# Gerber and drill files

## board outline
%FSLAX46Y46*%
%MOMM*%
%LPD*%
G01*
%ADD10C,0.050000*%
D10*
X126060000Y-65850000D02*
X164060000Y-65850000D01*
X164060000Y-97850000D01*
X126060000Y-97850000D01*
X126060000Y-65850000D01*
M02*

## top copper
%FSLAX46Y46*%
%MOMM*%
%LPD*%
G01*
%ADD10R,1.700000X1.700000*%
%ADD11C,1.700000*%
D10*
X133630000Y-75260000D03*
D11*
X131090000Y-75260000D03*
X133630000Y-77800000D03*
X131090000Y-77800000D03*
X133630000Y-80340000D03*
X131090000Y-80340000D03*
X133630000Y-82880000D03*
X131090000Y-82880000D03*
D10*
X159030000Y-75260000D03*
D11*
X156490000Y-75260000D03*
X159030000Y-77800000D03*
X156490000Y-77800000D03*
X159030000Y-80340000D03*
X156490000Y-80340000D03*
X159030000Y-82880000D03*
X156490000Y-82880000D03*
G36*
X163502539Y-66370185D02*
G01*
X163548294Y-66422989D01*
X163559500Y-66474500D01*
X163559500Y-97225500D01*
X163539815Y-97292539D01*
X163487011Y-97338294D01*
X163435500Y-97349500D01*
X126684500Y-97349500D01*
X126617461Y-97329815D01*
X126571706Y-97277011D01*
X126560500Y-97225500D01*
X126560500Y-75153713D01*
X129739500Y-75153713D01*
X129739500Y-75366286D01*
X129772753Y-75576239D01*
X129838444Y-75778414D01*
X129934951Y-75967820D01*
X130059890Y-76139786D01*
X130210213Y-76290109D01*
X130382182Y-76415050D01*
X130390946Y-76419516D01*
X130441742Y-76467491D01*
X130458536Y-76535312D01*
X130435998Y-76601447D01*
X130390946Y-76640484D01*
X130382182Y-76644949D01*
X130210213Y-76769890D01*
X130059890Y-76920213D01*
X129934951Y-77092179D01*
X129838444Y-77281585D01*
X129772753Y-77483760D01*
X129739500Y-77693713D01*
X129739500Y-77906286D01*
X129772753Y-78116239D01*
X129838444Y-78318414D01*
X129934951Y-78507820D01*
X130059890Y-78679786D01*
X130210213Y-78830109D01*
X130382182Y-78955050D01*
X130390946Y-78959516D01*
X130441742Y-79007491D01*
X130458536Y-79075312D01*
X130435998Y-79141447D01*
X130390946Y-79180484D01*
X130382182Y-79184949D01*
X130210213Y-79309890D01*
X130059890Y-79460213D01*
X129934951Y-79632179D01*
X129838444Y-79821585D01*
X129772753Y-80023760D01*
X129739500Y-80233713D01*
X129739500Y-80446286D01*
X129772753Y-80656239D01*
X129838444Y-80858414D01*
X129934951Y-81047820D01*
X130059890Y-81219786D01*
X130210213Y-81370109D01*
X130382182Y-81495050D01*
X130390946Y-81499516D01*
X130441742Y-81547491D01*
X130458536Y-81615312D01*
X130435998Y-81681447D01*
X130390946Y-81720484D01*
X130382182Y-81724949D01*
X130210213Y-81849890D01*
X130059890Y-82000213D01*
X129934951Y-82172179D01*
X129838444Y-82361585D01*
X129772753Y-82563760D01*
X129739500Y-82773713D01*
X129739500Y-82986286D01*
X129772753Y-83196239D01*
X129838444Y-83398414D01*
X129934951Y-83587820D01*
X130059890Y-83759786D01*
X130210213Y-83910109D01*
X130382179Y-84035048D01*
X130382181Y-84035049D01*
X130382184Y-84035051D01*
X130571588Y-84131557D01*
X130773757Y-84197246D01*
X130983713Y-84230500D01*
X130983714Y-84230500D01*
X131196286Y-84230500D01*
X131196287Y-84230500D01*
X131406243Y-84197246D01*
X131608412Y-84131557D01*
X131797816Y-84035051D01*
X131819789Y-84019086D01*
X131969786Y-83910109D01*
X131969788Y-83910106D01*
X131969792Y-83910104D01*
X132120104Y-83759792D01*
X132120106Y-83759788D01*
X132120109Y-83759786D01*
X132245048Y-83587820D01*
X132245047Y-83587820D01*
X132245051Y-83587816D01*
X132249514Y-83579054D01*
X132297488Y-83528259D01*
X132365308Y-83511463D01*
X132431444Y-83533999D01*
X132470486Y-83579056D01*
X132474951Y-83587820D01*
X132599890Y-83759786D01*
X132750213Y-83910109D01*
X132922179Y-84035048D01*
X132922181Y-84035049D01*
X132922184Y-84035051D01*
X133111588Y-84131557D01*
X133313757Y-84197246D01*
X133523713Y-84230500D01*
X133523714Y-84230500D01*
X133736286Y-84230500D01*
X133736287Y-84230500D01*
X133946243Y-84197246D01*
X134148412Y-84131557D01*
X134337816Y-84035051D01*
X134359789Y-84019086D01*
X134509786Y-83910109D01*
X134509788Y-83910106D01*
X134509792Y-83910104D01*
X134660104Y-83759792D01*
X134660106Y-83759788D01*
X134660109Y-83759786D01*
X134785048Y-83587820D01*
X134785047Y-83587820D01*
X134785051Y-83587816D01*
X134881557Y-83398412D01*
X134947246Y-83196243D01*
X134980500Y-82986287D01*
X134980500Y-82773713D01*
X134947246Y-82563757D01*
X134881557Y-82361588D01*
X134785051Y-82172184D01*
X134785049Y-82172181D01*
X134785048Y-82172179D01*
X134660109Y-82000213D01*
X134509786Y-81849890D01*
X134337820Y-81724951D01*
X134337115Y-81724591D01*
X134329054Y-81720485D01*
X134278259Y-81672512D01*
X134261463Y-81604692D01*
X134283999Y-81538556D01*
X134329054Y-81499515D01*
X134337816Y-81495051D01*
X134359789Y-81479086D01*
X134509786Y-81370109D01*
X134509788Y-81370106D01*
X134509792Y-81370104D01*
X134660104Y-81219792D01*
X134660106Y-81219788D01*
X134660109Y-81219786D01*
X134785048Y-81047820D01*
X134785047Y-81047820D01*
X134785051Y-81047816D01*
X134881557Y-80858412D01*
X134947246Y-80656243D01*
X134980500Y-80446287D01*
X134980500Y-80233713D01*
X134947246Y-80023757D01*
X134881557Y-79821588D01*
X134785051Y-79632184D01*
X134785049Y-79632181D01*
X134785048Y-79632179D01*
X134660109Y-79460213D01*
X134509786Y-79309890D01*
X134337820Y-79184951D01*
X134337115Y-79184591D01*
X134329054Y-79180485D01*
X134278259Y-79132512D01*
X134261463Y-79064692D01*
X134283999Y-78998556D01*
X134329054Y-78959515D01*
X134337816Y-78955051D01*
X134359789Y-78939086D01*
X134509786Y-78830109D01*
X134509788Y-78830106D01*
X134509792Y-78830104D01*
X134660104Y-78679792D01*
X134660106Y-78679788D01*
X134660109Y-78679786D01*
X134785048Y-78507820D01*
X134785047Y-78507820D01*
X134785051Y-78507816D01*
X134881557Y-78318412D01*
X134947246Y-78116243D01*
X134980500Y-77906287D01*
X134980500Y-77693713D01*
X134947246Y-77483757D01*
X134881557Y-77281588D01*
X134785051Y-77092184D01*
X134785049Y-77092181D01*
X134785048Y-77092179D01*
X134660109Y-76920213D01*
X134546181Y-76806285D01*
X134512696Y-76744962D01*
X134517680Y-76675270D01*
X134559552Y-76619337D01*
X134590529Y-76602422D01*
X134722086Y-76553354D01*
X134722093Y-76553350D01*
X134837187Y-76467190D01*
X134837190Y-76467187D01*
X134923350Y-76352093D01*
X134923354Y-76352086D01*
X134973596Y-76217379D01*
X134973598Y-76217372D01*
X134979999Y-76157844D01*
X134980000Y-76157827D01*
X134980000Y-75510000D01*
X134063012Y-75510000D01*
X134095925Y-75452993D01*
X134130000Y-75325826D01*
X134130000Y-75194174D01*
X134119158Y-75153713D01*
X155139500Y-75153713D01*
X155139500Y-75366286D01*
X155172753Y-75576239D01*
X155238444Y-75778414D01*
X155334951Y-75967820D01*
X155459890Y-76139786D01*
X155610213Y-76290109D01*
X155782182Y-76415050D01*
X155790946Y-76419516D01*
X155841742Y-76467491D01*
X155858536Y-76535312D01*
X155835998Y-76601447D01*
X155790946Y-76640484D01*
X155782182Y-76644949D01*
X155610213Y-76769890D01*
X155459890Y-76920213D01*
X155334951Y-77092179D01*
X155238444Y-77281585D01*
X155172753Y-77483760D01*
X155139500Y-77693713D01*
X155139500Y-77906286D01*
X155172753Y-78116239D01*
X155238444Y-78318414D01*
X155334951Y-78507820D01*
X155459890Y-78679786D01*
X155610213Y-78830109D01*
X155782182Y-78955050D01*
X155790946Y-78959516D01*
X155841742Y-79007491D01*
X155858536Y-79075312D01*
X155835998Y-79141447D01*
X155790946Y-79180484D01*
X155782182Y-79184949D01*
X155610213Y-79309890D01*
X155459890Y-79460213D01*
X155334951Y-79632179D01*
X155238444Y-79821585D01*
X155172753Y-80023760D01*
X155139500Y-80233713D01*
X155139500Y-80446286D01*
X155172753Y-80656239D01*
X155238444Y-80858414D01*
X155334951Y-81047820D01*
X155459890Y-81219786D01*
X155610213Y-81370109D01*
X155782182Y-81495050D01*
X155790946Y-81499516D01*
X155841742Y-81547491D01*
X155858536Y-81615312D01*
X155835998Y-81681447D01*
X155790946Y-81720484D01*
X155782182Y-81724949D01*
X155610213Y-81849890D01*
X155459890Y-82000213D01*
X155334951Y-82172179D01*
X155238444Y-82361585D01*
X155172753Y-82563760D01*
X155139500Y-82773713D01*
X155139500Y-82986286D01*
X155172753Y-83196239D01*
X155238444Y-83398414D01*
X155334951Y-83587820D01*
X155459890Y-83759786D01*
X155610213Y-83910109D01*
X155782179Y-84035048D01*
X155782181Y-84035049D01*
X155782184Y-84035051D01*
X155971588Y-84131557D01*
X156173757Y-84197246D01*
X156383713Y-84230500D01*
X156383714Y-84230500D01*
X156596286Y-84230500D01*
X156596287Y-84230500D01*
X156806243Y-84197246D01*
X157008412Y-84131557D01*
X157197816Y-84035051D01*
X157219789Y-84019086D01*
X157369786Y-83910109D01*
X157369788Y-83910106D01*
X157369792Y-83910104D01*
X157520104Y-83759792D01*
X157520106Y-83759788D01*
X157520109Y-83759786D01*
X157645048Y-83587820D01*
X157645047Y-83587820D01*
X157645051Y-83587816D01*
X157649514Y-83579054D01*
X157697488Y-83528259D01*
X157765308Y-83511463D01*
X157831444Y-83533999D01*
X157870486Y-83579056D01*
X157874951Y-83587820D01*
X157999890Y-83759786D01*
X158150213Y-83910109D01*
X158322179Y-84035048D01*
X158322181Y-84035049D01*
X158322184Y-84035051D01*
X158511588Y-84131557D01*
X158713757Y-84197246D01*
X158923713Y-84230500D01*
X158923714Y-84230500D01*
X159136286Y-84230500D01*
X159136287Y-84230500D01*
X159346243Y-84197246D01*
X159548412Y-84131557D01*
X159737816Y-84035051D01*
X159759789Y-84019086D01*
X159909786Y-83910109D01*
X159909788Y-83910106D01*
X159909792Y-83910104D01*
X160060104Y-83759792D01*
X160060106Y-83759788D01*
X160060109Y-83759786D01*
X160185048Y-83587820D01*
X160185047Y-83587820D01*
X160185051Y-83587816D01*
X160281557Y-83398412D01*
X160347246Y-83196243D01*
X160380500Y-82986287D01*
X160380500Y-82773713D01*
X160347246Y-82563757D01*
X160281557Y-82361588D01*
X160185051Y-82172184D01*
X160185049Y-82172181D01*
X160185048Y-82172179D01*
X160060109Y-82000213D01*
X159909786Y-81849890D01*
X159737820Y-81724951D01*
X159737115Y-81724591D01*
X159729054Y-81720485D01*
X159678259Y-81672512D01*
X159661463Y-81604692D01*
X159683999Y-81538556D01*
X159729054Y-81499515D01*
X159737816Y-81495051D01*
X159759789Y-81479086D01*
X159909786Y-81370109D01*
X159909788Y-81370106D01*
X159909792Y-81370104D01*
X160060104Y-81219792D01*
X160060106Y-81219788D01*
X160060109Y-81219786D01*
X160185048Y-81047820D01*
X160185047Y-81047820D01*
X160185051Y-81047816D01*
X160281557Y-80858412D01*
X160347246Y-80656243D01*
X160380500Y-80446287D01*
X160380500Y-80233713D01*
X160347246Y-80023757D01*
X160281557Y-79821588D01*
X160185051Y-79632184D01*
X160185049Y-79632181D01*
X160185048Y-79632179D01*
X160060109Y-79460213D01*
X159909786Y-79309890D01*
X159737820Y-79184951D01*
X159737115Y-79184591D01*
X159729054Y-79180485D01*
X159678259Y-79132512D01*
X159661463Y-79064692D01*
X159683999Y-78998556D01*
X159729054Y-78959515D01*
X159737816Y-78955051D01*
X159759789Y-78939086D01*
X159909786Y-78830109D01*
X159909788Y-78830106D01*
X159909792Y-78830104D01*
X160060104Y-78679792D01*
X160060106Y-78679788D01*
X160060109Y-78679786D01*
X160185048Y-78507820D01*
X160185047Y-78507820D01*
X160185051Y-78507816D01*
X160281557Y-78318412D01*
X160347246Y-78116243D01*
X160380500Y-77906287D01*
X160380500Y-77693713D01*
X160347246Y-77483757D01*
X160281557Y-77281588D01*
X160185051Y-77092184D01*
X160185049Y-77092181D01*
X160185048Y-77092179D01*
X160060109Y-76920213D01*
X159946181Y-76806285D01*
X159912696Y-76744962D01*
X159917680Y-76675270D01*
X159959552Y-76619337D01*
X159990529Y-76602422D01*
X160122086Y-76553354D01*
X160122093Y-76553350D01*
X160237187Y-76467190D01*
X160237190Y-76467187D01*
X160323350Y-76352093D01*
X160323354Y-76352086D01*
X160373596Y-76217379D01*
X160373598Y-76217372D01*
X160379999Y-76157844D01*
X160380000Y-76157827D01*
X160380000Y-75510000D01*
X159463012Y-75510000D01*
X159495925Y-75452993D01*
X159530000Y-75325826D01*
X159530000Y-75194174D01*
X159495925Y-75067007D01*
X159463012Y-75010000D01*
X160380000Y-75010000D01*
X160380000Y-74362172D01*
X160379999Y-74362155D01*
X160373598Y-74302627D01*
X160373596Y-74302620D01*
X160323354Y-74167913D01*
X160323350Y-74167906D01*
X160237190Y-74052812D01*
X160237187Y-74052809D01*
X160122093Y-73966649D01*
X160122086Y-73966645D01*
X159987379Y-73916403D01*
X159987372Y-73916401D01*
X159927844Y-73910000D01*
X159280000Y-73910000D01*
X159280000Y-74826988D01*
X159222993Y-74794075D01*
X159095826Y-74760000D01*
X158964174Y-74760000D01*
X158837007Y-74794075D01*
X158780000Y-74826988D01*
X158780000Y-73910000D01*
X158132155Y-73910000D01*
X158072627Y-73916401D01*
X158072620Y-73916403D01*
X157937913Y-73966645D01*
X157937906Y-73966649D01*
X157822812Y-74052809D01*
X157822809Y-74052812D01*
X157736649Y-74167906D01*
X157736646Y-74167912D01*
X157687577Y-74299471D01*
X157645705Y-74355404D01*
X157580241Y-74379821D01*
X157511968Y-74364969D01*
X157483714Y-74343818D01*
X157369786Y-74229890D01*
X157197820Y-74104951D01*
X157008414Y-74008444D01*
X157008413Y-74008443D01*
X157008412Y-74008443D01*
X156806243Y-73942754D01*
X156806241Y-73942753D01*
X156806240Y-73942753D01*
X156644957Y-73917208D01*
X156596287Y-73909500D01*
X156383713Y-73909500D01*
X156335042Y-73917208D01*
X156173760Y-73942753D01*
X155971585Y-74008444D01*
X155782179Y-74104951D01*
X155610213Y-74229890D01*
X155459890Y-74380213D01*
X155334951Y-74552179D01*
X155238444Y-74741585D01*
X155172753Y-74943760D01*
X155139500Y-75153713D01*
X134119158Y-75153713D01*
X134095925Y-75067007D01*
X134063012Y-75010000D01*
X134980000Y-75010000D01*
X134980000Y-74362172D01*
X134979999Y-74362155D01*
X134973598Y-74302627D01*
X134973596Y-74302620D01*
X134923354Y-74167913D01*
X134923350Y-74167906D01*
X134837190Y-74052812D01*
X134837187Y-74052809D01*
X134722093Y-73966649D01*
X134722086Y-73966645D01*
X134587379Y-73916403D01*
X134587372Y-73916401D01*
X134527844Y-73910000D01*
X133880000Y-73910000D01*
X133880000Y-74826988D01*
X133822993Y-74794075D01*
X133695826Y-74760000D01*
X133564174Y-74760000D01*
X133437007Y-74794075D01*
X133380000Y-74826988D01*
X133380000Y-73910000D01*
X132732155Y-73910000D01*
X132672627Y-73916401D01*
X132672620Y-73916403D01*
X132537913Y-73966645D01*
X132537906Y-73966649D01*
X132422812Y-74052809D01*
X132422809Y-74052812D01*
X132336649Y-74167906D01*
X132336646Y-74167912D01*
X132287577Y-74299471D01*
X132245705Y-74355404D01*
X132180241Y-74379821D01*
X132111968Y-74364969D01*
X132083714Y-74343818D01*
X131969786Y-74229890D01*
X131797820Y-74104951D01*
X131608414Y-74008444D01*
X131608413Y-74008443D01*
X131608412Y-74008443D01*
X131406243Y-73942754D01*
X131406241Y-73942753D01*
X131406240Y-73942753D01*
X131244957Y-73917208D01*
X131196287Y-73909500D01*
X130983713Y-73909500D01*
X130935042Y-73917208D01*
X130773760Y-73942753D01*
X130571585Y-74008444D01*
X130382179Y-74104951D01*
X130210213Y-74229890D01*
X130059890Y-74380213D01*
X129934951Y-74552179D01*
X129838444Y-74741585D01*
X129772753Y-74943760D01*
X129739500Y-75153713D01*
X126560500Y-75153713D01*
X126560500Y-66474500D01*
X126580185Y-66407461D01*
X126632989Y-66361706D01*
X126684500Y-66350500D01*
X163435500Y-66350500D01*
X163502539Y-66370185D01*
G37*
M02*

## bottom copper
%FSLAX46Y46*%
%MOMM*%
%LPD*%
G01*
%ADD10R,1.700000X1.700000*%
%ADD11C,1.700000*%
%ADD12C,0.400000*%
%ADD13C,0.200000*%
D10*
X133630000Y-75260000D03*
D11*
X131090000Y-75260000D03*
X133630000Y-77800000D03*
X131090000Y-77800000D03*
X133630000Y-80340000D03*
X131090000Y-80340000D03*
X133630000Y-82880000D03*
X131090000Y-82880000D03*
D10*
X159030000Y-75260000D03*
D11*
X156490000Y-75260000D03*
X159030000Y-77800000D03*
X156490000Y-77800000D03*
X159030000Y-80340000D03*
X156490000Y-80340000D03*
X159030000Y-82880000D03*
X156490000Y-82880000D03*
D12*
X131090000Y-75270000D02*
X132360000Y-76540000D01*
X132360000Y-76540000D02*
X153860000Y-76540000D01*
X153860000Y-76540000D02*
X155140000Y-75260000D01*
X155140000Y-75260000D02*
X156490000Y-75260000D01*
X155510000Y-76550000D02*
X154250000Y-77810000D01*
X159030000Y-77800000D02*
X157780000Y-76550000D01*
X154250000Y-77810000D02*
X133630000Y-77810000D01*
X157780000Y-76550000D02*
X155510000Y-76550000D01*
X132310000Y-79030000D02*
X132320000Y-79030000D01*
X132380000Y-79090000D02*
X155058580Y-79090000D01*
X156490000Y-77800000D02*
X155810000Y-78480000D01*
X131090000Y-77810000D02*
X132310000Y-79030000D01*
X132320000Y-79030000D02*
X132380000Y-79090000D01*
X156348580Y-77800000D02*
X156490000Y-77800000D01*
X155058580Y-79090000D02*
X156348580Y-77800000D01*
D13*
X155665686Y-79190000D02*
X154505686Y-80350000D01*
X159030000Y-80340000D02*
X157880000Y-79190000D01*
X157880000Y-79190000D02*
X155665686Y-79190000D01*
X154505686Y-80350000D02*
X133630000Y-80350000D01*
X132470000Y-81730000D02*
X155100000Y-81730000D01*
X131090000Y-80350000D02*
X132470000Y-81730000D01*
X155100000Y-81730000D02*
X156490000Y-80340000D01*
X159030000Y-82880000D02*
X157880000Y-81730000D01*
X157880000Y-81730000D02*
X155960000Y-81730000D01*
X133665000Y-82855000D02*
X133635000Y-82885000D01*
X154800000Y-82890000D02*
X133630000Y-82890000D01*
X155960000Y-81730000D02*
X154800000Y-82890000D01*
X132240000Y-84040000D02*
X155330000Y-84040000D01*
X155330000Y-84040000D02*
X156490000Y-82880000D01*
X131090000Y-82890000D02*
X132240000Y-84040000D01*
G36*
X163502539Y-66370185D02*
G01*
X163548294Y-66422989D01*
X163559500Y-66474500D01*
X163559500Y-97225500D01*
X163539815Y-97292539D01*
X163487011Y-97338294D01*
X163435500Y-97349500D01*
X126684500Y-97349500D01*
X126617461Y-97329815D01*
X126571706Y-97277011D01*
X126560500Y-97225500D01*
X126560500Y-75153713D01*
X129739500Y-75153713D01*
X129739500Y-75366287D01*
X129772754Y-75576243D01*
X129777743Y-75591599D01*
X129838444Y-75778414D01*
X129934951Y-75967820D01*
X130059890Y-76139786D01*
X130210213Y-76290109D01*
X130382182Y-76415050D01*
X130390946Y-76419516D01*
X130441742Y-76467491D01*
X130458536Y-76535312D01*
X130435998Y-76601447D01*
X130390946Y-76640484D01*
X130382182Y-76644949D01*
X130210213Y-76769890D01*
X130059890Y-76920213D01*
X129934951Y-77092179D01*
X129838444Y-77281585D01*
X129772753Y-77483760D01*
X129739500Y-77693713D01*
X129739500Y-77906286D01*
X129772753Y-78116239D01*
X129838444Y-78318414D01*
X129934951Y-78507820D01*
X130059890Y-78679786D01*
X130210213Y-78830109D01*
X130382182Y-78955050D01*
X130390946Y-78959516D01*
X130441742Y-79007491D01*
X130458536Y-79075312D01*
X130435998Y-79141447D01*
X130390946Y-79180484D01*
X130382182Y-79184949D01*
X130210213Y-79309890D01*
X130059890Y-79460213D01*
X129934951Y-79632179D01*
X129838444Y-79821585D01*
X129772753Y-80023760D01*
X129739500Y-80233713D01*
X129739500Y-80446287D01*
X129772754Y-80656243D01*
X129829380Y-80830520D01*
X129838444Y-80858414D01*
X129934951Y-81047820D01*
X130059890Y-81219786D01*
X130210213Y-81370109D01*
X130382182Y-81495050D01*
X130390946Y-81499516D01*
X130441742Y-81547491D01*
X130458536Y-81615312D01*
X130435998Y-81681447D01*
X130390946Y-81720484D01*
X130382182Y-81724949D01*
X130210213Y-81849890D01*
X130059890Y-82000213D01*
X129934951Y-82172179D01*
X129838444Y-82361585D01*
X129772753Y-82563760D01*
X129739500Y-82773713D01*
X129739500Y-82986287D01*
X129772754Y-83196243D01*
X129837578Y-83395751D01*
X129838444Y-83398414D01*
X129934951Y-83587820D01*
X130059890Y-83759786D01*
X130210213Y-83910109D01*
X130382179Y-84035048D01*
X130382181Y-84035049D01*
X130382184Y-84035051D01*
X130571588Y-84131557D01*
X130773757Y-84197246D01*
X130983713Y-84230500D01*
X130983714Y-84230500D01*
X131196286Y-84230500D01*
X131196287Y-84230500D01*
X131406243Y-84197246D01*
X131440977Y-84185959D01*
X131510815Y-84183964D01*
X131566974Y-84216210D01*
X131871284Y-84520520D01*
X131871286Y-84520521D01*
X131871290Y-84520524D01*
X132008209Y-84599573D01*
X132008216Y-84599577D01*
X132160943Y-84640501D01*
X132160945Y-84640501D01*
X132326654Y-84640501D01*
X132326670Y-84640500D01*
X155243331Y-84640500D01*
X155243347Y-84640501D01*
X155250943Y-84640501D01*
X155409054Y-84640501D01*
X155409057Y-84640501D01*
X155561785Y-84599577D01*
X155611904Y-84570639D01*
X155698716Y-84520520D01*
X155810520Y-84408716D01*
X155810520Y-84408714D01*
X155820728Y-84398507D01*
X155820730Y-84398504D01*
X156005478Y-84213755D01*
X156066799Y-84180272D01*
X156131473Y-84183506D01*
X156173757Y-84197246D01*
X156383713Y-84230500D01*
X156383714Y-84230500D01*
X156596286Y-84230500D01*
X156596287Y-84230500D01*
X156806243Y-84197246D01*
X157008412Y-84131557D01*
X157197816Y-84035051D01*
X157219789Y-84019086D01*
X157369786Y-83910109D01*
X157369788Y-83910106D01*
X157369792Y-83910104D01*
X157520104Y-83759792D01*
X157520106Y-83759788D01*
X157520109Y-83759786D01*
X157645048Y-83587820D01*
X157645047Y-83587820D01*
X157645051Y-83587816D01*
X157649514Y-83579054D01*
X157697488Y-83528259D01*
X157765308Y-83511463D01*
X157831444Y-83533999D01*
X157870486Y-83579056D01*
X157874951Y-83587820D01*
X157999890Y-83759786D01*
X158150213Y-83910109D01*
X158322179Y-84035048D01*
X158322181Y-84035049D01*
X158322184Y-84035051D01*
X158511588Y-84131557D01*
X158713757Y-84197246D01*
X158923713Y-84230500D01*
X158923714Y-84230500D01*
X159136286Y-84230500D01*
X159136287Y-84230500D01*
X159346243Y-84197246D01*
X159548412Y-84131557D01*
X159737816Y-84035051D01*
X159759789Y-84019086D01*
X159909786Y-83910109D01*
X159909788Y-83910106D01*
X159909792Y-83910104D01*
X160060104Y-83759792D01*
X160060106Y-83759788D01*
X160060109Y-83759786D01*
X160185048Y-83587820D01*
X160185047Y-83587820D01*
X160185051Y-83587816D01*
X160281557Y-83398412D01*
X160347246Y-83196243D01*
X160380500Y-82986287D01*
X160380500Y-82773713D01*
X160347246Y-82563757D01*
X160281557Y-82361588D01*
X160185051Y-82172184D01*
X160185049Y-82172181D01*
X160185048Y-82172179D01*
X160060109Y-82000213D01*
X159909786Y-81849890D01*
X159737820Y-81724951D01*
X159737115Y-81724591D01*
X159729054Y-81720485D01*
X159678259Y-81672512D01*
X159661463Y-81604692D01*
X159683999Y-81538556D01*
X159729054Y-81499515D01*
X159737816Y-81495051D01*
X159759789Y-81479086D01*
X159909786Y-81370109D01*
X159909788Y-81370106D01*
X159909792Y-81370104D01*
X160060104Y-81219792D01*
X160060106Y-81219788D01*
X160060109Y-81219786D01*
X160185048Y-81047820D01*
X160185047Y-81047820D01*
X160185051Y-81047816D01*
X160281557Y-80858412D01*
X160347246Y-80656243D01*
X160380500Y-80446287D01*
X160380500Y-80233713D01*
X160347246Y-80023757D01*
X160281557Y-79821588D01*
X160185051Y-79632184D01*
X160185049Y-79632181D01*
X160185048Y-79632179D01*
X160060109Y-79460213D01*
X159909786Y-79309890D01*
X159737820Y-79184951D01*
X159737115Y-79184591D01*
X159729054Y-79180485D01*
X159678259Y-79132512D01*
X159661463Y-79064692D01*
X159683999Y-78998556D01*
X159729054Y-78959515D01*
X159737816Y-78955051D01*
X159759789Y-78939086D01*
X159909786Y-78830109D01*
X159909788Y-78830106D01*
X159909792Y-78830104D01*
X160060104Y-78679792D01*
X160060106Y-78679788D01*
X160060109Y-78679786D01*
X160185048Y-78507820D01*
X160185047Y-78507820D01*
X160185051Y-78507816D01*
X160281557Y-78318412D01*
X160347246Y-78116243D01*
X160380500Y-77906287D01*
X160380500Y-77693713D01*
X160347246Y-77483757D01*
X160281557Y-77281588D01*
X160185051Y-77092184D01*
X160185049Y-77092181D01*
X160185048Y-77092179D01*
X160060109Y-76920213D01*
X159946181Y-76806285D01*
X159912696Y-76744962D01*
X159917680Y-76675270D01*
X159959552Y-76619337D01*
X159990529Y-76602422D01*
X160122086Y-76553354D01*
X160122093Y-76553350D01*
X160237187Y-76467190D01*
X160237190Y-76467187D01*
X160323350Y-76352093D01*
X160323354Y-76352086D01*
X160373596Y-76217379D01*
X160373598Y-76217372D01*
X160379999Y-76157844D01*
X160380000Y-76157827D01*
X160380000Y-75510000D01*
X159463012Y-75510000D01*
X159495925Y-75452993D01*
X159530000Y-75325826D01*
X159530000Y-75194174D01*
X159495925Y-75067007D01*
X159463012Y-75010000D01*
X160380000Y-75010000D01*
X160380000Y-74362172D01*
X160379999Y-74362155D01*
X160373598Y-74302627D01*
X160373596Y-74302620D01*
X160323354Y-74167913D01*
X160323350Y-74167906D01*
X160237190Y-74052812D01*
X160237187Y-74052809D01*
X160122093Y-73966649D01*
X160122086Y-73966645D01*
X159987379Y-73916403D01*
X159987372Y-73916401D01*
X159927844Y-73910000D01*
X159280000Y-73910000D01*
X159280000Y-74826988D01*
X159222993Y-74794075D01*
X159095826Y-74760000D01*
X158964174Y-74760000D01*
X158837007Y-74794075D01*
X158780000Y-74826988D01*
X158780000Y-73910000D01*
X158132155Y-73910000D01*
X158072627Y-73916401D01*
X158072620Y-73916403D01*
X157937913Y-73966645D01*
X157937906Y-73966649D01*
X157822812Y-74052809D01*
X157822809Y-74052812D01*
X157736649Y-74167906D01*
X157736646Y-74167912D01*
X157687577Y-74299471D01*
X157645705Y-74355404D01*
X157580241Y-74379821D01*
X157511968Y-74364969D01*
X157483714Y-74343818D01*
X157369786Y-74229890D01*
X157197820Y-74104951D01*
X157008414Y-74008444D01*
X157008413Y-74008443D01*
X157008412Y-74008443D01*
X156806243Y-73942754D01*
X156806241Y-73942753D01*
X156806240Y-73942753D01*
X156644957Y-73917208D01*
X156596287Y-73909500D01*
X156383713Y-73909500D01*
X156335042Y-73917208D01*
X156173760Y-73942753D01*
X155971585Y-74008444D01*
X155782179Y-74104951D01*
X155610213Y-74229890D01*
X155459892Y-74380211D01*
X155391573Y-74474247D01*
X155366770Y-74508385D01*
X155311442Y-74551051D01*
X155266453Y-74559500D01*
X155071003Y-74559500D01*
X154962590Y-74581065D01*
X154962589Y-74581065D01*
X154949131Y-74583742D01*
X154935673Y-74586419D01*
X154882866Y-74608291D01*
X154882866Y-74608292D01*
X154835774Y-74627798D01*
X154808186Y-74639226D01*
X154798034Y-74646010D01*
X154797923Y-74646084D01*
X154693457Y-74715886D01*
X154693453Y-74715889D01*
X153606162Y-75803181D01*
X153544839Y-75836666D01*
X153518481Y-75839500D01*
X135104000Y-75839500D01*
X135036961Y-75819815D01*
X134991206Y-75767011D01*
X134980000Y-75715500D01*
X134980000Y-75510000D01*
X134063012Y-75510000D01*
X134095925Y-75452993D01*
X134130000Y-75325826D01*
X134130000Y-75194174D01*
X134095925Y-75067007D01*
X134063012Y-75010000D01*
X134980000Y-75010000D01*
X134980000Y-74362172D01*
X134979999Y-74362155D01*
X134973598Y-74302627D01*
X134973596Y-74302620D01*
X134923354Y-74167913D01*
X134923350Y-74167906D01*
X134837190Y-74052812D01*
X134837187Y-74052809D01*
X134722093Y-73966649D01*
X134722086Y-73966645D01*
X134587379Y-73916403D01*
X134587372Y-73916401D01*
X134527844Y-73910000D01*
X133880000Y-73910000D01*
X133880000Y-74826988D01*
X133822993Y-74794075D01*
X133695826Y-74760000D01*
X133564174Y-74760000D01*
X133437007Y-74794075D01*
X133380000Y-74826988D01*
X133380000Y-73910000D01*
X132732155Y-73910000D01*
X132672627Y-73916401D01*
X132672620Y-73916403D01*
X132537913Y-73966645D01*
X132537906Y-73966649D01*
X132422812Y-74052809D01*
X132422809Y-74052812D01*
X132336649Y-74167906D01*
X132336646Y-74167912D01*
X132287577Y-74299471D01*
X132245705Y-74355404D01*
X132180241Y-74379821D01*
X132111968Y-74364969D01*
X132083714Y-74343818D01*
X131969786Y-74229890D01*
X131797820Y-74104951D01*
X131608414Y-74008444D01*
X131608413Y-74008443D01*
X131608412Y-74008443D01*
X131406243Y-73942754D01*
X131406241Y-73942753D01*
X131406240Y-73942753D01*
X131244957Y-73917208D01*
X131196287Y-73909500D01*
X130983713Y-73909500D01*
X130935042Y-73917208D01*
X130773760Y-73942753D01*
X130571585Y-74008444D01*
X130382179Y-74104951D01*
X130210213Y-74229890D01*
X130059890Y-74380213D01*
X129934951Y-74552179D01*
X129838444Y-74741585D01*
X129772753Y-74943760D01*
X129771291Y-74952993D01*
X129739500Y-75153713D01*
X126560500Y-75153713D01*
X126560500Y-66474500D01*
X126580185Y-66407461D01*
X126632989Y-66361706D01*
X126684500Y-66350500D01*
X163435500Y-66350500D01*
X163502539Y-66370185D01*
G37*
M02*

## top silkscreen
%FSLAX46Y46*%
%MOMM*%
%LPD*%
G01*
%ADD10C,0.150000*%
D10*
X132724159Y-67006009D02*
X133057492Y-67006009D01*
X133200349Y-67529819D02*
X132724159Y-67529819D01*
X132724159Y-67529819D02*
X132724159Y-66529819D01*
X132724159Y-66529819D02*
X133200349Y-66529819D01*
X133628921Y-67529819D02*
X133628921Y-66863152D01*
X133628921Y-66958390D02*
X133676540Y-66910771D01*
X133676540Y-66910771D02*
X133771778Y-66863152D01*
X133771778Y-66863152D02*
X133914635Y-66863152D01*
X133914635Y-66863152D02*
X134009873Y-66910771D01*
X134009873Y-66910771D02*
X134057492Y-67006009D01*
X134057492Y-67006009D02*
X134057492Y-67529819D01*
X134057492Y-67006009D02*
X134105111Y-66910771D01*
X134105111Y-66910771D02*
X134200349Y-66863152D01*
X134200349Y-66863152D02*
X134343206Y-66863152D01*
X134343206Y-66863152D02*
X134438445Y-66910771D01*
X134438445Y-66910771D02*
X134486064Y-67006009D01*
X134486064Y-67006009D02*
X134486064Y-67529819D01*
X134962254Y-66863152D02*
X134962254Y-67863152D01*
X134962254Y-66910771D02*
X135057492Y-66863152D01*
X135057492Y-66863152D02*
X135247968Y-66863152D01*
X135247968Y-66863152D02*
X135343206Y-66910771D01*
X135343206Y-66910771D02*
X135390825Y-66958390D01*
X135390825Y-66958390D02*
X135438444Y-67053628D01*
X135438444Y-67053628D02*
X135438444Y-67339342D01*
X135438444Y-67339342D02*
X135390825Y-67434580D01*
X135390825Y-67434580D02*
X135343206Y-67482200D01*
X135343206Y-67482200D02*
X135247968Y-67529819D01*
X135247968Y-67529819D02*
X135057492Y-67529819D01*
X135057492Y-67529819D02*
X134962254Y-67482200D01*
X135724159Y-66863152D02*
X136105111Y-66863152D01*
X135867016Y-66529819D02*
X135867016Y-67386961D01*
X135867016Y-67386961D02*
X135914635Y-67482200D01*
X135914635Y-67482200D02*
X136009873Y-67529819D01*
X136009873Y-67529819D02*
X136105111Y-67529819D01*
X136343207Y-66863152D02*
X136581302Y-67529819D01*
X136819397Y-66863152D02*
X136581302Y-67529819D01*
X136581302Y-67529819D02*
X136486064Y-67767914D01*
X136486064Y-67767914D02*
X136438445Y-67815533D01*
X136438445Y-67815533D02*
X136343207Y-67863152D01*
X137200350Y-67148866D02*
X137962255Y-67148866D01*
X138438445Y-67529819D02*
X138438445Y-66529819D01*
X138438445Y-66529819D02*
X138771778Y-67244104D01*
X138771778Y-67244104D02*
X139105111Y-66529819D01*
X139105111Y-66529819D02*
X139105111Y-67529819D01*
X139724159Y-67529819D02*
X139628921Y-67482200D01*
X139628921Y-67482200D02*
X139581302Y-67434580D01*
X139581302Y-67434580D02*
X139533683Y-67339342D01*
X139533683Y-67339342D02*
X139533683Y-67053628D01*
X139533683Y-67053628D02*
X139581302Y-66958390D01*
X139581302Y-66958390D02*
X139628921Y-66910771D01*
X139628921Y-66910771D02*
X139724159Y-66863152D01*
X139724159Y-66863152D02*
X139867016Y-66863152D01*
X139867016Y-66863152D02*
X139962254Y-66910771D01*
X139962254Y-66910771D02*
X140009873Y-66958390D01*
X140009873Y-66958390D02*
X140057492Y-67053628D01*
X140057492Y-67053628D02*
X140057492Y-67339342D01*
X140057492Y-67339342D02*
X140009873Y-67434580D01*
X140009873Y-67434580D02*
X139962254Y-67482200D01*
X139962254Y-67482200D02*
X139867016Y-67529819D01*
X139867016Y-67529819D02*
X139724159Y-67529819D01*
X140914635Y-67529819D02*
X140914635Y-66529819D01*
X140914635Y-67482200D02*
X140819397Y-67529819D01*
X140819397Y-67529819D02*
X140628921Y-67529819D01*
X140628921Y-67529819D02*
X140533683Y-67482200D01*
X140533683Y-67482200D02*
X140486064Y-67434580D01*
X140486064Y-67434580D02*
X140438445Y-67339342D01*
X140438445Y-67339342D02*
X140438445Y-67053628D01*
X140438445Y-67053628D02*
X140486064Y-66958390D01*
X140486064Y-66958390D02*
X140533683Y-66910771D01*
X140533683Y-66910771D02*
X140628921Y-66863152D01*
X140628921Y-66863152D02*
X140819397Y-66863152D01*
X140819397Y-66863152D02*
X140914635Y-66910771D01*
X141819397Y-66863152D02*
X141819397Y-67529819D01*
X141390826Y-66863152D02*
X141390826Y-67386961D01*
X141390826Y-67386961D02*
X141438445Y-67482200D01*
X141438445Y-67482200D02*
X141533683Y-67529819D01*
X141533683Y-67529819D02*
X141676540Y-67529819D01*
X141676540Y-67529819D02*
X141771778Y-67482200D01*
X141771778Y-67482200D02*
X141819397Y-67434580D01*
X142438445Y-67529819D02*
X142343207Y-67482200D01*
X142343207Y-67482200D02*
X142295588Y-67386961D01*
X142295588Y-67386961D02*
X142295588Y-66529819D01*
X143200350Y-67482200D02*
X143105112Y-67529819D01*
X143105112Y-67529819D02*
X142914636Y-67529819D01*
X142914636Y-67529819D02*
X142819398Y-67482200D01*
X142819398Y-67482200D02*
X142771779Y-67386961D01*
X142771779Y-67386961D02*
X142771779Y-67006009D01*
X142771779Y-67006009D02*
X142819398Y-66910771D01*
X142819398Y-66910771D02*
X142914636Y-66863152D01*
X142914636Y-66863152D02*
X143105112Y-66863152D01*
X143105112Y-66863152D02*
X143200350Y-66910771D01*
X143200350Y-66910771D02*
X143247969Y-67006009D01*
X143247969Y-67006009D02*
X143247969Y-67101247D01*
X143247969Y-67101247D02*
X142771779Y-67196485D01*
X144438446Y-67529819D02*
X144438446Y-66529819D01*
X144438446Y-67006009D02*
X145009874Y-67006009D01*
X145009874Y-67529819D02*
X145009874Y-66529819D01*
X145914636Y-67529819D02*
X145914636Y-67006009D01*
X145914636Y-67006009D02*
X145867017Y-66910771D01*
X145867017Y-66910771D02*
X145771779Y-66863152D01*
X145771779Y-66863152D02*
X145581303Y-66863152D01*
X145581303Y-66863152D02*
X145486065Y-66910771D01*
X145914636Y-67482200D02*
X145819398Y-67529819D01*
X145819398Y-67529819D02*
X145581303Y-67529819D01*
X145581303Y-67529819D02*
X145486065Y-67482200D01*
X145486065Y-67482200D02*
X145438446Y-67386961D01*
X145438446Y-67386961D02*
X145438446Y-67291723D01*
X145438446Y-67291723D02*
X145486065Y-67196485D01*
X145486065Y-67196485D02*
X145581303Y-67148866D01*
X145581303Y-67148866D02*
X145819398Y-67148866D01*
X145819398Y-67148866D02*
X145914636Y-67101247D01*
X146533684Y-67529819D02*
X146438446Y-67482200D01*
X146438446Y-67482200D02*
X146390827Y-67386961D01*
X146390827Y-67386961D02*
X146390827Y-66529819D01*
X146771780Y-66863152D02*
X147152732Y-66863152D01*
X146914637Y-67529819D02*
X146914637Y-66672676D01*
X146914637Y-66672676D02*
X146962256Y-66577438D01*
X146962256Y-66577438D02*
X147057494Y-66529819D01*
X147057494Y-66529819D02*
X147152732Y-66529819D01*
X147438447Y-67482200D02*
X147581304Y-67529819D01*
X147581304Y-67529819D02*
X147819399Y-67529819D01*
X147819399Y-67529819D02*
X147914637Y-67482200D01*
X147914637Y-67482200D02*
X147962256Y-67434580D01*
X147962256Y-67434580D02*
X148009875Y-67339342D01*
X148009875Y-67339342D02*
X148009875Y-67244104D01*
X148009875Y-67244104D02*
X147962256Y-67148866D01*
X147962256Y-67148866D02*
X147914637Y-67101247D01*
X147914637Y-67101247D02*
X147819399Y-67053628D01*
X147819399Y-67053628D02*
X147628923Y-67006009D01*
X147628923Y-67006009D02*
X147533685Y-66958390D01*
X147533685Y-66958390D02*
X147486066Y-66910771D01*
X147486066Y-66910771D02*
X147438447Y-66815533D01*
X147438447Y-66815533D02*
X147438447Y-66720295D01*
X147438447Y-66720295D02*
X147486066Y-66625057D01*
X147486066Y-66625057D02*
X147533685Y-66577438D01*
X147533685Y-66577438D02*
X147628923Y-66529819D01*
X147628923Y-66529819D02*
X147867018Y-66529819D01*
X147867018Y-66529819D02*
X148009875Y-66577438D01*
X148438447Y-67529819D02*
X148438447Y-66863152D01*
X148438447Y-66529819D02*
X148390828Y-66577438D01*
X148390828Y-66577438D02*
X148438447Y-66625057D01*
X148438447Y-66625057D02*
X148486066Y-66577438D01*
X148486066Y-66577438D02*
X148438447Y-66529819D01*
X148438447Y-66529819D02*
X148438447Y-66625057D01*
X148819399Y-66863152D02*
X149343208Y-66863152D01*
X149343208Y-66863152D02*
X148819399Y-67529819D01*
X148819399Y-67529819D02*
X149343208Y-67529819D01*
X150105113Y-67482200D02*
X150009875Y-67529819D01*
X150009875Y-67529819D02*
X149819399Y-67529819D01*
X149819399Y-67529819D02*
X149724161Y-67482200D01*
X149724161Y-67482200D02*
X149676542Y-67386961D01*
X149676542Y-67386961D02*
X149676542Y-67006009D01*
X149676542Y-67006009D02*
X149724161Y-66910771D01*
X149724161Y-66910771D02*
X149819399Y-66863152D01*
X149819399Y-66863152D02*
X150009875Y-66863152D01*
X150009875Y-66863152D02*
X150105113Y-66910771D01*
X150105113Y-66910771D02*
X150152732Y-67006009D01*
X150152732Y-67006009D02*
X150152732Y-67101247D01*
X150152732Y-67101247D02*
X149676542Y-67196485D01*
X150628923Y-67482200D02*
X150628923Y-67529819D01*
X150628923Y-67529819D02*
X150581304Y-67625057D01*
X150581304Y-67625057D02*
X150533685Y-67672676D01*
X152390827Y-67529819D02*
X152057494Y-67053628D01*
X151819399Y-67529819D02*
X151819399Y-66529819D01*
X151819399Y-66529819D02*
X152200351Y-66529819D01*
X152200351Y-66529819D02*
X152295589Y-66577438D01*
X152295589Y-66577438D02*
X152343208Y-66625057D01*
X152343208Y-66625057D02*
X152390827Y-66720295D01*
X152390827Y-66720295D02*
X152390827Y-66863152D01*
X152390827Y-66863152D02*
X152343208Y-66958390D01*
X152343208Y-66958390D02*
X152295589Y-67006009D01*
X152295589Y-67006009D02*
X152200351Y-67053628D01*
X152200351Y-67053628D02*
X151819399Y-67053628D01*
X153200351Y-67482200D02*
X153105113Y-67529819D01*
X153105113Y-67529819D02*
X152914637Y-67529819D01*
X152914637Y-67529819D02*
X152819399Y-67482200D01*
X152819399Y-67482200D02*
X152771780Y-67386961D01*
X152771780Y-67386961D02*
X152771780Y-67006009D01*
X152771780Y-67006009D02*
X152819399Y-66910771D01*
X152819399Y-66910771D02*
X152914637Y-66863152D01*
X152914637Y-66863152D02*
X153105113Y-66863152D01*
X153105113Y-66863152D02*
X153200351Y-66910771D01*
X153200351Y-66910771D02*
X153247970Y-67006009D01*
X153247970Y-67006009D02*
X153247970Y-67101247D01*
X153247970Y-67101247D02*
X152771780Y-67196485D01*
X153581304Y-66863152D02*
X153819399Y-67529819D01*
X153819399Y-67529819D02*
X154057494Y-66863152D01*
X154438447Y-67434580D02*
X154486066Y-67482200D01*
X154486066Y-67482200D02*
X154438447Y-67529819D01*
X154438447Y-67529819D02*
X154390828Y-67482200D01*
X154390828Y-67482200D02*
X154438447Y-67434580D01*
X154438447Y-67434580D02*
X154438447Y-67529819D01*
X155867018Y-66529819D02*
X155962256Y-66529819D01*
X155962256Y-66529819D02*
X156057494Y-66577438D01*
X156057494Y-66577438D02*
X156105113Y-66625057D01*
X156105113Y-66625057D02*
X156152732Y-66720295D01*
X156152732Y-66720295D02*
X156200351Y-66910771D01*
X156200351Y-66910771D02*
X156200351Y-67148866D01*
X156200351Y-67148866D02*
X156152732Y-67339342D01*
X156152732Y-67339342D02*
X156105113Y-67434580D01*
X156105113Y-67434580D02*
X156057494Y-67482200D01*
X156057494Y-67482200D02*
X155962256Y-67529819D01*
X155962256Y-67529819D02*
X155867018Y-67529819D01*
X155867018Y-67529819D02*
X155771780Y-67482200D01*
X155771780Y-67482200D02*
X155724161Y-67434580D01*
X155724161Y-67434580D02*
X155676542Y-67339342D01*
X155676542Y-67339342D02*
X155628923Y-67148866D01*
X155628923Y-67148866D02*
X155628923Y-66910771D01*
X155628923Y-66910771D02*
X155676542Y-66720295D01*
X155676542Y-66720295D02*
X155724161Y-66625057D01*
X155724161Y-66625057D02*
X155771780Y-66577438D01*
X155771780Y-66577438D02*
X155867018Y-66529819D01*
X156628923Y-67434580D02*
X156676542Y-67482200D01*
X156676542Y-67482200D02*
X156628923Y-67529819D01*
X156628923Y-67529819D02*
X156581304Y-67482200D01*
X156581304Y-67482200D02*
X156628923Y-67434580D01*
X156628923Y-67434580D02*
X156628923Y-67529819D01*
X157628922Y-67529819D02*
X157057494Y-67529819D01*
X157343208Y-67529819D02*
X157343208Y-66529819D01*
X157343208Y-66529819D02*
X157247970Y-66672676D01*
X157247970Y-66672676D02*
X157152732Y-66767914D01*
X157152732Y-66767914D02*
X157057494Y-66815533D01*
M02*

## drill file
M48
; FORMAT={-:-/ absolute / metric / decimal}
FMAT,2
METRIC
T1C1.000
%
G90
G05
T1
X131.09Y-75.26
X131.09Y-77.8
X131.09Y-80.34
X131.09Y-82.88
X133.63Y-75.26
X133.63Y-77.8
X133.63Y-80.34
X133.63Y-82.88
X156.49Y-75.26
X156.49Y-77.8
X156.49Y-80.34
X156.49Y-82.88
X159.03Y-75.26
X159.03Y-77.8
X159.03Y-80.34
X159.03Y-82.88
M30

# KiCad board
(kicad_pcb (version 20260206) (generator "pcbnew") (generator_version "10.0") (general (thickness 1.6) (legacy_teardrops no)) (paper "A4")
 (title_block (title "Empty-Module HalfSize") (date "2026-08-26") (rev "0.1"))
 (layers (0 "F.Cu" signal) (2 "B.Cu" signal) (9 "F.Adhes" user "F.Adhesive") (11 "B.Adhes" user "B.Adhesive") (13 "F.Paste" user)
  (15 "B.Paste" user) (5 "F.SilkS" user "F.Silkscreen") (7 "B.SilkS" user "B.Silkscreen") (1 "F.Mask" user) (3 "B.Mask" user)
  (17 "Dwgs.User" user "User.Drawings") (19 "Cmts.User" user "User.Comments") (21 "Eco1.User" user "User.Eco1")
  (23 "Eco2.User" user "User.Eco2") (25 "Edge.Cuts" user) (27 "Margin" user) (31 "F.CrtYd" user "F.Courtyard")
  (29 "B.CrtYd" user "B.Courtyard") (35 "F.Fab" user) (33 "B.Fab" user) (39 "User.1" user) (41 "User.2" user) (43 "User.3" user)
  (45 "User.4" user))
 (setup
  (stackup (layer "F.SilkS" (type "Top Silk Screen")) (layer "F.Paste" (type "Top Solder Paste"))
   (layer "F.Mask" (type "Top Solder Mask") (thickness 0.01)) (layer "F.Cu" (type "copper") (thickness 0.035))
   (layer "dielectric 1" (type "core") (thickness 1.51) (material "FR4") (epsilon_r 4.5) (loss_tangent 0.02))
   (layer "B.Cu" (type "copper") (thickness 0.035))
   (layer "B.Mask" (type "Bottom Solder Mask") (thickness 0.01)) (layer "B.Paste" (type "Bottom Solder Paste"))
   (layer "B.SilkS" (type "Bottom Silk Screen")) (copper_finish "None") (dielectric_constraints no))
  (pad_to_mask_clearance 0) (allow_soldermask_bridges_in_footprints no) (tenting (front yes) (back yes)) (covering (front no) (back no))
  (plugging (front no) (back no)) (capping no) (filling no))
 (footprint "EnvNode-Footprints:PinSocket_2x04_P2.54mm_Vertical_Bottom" (layer "B.Cu") (at 131.09 75.26 180)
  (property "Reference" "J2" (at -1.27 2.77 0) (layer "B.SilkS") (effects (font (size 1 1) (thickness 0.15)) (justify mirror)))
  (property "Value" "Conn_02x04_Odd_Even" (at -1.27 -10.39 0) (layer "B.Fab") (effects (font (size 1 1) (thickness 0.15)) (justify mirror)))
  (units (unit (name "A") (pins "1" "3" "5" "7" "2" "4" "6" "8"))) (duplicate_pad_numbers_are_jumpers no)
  (pad "1" thru_hole rect (at -2.54 0 180) (size 1.7 1.7) (drill 1) (layers "*.Cu" "*.Mask") (remove_unused_layers no) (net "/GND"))
  (pad "2" thru_hole circle (at 0 0 180) (size 1.7 1.7) (drill 1) (layers "*.Cu" "*.Mask") (remove_unused_layers no) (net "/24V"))
  (pad "3" thru_hole circle (at -2.54 -2.54 180) (size 1.7 1.7) (drill 1) (layers "*.Cu" "*.Mask") (remove_unused_layers no) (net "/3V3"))
  (pad "4" thru_hole circle (at 0 -2.54 180) (size 1.7 1.7) (drill 1) (layers "*.Cu" "*.Mask") (remove_unused_layers no) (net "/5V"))
  (pad "5" thru_hole circle (at -2.54 -5.08 180) (size 1.7 1.7) (drill 1) (layers "*.Cu" "*.Mask") (remove_unused_layers no) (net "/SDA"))
  (pad "6" thru_hole circle (at 0 -5.08 180) (size 1.7 1.7) (drill 1) (layers "*.Cu" "*.Mask") (remove_unused_layers no) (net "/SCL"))
  (pad "7" thru_hole circle (at -2.54 -7.62 180) (size 1.7 1.7) (drill 1) (layers "*.Cu" "*.Mask") (remove_unused_layers no) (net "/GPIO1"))
  (pad "8" thru_hole circle (at 0 -7.62 180) (size 1.7 1.7) (drill 1) (layers "*.Cu" "*.Mask") (remove_unused_layers no) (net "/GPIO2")))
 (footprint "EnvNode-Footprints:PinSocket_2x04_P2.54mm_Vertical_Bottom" (layer "B.Cu") (at 156.49 75.26 180)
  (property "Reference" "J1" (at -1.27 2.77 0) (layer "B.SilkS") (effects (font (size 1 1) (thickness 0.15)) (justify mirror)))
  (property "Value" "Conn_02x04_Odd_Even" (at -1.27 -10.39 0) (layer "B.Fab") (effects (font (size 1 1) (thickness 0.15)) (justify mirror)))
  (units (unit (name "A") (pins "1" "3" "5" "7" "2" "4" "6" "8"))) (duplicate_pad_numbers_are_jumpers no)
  (pad "1" thru_hole rect (at -2.54 0 180) (size 1.7 1.7) (drill 1) (layers "*.Cu" "*.Mask") (remove_unused_layers no) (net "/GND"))
  (pad "2" thru_hole circle (at 0 0 180) (size 1.7 1.7) (drill 1) (layers "*.Cu" "*.Mask") (remove_unused_layers no) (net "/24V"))
  (pad "3" thru_hole circle (at -2.54 -2.54 180) (size 1.7 1.7) (drill 1) (layers "*.Cu" "*.Mask") (remove_unused_layers no) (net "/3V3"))
  (pad "4" thru_hole circle (at 0 -2.54 180) (size 1.7 1.7) (drill 1) (layers "*.Cu" "*.Mask") (remove_unused_layers no) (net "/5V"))
  (pad "5" thru_hole circle (at -2.54 -5.08 180) (size 1.7 1.7) (drill 1) (layers "*.Cu" "*.Mask") (remove_unused_layers no) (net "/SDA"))
  (pad "6" thru_hole circle (at 0 -5.08 180) (size 1.7 1.7) (drill 1) (layers "*.Cu" "*.Mask") (remove_unused_layers no) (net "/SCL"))
  (pad "7" thru_hole circle (at -2.54 -7.62 180) (size 1.7 1.7) (drill 1) (layers "*.Cu" "*.Mask") (remove_unused_layers no) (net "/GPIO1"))
  (pad "8" thru_hole circle (at 0 -7.62 180) (size 1.7 1.7) (drill 1) (layers "*.Cu" "*.Mask") (remove_unused_layers no) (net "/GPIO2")))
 (gr_rect (start 126.06 65.85) (end 164.06 97.85) (stroke (width 0.05) (type solid)) (fill no) (layer "Edge.Cuts"))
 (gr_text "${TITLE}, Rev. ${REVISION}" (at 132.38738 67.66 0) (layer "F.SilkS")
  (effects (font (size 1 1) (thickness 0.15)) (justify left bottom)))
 (segment (start 131.09 75.27) (end 132.36 76.54) (width 0.4) (layer "B.Cu") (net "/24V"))
 (segment (start 132.36 76.54) (end 153.86 76.54) (width 0.4) (layer "B.Cu") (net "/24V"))
 (segment (start 153.86 76.54) (end 155.14 75.26) (width 0.4) (layer "B.Cu") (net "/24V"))
 (segment (start 155.14 75.26) (end 156.49 75.26) (width 0.4) (layer "B.Cu") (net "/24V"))
 (segment (start 155.51 76.55) (end 154.25 77.81) (width 0.4) (layer "B.Cu") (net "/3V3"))
 (segment (start 159.03 77.8) (end 157.78 76.55) (width 0.4) (layer "B.Cu") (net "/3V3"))
 (segment (start 154.25 77.81) (end 133.63 77.81) (width 0.4) (layer "B.Cu") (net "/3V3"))
 (segment (start 157.78 76.55) (end 155.51 76.55) (width 0.4) (layer "B.Cu") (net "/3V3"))
 (segment (start 132.31 79.03) (end 132.32 79.03) (width 0.4) (layer "B.Cu") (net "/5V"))
 (segment (start 132.38 79.09) (end 155.05858 79.09) (width 0.4) (layer "B.Cu") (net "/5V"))
 (segment (start 156.49 77.8) (end 155.81 78.48) (width 0.4) (layer "B.Cu") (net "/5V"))
 (segment (start 131.09 77.81) (end 132.31 79.03) (width 0.4) (layer "B.Cu") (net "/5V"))
 (segment (start 132.32 79.03) (end 132.38 79.09) (width 0.4) (layer "B.Cu") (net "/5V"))
 (segment (start 156.34858 77.8) (end 156.49 77.8) (width 0.4) (layer "B.Cu") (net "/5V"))
 (segment (start 155.05858 79.09) (end 156.34858 77.8) (width 0.4) (layer "B.Cu") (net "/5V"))
 (segment (start 155.665686 79.19) (end 154.505686 80.35) (width 0.2) (layer "B.Cu") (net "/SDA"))
 (segment (start 159.03 80.34) (end 157.88 79.19) (width 0.2) (layer "B.Cu") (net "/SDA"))
 (segment (start 157.88 79.19) (end 155.665686 79.19) (width 0.2) (layer "B.Cu") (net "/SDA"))
 (segment (start 154.505686 80.35) (end 133.63 80.35) (width 0.2) (layer "B.Cu") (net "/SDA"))
 (segment (start 132.47 81.73) (end 155.1 81.73) (width 0.2) (layer "B.Cu") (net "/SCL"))
 (segment (start 131.09 80.35) (end 132.47 81.73) (width 0.2) (layer "B.Cu") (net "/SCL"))
 (segment (start 155.1 81.73) (end 156.49 80.34) (width 0.2) (layer "B.Cu") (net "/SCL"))
 (segment (start 159.03 82.88) (end 157.88 81.73) (width 0.2) (layer "B.Cu") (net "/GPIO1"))
 (segment (start 157.88 81.73) (end 155.96 81.73) (width 0.2) (layer "B.Cu") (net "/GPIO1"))
 (segment (start 133.665 82.855) (end 133.635 82.885) (width 0.2) (layer "B.Cu") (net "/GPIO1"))
 (segment (start 154.8 82.89) (end 133.63 82.89) (width 0.2) (layer "B.Cu") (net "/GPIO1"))
 (segment (start 155.96 81.73) (end 154.8 82.89) (width 0.2) (layer "B.Cu") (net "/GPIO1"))
 (segment (start 132.24 84.04) (end 155.33 84.04) (width 0.2) (layer "B.Cu") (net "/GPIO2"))
 (segment (start 155.33 84.04) (end 156.49 82.88) (width 0.2) (layer "B.Cu") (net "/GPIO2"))
 (segment (start 131.09 82.89) (end 132.24 84.04) (width 0.2) (layer "B.Cu") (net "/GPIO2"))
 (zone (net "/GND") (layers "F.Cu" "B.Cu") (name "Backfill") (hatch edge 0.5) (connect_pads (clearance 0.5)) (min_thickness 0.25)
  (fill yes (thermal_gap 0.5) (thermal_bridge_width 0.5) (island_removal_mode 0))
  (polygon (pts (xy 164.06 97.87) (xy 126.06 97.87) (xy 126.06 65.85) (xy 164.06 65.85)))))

